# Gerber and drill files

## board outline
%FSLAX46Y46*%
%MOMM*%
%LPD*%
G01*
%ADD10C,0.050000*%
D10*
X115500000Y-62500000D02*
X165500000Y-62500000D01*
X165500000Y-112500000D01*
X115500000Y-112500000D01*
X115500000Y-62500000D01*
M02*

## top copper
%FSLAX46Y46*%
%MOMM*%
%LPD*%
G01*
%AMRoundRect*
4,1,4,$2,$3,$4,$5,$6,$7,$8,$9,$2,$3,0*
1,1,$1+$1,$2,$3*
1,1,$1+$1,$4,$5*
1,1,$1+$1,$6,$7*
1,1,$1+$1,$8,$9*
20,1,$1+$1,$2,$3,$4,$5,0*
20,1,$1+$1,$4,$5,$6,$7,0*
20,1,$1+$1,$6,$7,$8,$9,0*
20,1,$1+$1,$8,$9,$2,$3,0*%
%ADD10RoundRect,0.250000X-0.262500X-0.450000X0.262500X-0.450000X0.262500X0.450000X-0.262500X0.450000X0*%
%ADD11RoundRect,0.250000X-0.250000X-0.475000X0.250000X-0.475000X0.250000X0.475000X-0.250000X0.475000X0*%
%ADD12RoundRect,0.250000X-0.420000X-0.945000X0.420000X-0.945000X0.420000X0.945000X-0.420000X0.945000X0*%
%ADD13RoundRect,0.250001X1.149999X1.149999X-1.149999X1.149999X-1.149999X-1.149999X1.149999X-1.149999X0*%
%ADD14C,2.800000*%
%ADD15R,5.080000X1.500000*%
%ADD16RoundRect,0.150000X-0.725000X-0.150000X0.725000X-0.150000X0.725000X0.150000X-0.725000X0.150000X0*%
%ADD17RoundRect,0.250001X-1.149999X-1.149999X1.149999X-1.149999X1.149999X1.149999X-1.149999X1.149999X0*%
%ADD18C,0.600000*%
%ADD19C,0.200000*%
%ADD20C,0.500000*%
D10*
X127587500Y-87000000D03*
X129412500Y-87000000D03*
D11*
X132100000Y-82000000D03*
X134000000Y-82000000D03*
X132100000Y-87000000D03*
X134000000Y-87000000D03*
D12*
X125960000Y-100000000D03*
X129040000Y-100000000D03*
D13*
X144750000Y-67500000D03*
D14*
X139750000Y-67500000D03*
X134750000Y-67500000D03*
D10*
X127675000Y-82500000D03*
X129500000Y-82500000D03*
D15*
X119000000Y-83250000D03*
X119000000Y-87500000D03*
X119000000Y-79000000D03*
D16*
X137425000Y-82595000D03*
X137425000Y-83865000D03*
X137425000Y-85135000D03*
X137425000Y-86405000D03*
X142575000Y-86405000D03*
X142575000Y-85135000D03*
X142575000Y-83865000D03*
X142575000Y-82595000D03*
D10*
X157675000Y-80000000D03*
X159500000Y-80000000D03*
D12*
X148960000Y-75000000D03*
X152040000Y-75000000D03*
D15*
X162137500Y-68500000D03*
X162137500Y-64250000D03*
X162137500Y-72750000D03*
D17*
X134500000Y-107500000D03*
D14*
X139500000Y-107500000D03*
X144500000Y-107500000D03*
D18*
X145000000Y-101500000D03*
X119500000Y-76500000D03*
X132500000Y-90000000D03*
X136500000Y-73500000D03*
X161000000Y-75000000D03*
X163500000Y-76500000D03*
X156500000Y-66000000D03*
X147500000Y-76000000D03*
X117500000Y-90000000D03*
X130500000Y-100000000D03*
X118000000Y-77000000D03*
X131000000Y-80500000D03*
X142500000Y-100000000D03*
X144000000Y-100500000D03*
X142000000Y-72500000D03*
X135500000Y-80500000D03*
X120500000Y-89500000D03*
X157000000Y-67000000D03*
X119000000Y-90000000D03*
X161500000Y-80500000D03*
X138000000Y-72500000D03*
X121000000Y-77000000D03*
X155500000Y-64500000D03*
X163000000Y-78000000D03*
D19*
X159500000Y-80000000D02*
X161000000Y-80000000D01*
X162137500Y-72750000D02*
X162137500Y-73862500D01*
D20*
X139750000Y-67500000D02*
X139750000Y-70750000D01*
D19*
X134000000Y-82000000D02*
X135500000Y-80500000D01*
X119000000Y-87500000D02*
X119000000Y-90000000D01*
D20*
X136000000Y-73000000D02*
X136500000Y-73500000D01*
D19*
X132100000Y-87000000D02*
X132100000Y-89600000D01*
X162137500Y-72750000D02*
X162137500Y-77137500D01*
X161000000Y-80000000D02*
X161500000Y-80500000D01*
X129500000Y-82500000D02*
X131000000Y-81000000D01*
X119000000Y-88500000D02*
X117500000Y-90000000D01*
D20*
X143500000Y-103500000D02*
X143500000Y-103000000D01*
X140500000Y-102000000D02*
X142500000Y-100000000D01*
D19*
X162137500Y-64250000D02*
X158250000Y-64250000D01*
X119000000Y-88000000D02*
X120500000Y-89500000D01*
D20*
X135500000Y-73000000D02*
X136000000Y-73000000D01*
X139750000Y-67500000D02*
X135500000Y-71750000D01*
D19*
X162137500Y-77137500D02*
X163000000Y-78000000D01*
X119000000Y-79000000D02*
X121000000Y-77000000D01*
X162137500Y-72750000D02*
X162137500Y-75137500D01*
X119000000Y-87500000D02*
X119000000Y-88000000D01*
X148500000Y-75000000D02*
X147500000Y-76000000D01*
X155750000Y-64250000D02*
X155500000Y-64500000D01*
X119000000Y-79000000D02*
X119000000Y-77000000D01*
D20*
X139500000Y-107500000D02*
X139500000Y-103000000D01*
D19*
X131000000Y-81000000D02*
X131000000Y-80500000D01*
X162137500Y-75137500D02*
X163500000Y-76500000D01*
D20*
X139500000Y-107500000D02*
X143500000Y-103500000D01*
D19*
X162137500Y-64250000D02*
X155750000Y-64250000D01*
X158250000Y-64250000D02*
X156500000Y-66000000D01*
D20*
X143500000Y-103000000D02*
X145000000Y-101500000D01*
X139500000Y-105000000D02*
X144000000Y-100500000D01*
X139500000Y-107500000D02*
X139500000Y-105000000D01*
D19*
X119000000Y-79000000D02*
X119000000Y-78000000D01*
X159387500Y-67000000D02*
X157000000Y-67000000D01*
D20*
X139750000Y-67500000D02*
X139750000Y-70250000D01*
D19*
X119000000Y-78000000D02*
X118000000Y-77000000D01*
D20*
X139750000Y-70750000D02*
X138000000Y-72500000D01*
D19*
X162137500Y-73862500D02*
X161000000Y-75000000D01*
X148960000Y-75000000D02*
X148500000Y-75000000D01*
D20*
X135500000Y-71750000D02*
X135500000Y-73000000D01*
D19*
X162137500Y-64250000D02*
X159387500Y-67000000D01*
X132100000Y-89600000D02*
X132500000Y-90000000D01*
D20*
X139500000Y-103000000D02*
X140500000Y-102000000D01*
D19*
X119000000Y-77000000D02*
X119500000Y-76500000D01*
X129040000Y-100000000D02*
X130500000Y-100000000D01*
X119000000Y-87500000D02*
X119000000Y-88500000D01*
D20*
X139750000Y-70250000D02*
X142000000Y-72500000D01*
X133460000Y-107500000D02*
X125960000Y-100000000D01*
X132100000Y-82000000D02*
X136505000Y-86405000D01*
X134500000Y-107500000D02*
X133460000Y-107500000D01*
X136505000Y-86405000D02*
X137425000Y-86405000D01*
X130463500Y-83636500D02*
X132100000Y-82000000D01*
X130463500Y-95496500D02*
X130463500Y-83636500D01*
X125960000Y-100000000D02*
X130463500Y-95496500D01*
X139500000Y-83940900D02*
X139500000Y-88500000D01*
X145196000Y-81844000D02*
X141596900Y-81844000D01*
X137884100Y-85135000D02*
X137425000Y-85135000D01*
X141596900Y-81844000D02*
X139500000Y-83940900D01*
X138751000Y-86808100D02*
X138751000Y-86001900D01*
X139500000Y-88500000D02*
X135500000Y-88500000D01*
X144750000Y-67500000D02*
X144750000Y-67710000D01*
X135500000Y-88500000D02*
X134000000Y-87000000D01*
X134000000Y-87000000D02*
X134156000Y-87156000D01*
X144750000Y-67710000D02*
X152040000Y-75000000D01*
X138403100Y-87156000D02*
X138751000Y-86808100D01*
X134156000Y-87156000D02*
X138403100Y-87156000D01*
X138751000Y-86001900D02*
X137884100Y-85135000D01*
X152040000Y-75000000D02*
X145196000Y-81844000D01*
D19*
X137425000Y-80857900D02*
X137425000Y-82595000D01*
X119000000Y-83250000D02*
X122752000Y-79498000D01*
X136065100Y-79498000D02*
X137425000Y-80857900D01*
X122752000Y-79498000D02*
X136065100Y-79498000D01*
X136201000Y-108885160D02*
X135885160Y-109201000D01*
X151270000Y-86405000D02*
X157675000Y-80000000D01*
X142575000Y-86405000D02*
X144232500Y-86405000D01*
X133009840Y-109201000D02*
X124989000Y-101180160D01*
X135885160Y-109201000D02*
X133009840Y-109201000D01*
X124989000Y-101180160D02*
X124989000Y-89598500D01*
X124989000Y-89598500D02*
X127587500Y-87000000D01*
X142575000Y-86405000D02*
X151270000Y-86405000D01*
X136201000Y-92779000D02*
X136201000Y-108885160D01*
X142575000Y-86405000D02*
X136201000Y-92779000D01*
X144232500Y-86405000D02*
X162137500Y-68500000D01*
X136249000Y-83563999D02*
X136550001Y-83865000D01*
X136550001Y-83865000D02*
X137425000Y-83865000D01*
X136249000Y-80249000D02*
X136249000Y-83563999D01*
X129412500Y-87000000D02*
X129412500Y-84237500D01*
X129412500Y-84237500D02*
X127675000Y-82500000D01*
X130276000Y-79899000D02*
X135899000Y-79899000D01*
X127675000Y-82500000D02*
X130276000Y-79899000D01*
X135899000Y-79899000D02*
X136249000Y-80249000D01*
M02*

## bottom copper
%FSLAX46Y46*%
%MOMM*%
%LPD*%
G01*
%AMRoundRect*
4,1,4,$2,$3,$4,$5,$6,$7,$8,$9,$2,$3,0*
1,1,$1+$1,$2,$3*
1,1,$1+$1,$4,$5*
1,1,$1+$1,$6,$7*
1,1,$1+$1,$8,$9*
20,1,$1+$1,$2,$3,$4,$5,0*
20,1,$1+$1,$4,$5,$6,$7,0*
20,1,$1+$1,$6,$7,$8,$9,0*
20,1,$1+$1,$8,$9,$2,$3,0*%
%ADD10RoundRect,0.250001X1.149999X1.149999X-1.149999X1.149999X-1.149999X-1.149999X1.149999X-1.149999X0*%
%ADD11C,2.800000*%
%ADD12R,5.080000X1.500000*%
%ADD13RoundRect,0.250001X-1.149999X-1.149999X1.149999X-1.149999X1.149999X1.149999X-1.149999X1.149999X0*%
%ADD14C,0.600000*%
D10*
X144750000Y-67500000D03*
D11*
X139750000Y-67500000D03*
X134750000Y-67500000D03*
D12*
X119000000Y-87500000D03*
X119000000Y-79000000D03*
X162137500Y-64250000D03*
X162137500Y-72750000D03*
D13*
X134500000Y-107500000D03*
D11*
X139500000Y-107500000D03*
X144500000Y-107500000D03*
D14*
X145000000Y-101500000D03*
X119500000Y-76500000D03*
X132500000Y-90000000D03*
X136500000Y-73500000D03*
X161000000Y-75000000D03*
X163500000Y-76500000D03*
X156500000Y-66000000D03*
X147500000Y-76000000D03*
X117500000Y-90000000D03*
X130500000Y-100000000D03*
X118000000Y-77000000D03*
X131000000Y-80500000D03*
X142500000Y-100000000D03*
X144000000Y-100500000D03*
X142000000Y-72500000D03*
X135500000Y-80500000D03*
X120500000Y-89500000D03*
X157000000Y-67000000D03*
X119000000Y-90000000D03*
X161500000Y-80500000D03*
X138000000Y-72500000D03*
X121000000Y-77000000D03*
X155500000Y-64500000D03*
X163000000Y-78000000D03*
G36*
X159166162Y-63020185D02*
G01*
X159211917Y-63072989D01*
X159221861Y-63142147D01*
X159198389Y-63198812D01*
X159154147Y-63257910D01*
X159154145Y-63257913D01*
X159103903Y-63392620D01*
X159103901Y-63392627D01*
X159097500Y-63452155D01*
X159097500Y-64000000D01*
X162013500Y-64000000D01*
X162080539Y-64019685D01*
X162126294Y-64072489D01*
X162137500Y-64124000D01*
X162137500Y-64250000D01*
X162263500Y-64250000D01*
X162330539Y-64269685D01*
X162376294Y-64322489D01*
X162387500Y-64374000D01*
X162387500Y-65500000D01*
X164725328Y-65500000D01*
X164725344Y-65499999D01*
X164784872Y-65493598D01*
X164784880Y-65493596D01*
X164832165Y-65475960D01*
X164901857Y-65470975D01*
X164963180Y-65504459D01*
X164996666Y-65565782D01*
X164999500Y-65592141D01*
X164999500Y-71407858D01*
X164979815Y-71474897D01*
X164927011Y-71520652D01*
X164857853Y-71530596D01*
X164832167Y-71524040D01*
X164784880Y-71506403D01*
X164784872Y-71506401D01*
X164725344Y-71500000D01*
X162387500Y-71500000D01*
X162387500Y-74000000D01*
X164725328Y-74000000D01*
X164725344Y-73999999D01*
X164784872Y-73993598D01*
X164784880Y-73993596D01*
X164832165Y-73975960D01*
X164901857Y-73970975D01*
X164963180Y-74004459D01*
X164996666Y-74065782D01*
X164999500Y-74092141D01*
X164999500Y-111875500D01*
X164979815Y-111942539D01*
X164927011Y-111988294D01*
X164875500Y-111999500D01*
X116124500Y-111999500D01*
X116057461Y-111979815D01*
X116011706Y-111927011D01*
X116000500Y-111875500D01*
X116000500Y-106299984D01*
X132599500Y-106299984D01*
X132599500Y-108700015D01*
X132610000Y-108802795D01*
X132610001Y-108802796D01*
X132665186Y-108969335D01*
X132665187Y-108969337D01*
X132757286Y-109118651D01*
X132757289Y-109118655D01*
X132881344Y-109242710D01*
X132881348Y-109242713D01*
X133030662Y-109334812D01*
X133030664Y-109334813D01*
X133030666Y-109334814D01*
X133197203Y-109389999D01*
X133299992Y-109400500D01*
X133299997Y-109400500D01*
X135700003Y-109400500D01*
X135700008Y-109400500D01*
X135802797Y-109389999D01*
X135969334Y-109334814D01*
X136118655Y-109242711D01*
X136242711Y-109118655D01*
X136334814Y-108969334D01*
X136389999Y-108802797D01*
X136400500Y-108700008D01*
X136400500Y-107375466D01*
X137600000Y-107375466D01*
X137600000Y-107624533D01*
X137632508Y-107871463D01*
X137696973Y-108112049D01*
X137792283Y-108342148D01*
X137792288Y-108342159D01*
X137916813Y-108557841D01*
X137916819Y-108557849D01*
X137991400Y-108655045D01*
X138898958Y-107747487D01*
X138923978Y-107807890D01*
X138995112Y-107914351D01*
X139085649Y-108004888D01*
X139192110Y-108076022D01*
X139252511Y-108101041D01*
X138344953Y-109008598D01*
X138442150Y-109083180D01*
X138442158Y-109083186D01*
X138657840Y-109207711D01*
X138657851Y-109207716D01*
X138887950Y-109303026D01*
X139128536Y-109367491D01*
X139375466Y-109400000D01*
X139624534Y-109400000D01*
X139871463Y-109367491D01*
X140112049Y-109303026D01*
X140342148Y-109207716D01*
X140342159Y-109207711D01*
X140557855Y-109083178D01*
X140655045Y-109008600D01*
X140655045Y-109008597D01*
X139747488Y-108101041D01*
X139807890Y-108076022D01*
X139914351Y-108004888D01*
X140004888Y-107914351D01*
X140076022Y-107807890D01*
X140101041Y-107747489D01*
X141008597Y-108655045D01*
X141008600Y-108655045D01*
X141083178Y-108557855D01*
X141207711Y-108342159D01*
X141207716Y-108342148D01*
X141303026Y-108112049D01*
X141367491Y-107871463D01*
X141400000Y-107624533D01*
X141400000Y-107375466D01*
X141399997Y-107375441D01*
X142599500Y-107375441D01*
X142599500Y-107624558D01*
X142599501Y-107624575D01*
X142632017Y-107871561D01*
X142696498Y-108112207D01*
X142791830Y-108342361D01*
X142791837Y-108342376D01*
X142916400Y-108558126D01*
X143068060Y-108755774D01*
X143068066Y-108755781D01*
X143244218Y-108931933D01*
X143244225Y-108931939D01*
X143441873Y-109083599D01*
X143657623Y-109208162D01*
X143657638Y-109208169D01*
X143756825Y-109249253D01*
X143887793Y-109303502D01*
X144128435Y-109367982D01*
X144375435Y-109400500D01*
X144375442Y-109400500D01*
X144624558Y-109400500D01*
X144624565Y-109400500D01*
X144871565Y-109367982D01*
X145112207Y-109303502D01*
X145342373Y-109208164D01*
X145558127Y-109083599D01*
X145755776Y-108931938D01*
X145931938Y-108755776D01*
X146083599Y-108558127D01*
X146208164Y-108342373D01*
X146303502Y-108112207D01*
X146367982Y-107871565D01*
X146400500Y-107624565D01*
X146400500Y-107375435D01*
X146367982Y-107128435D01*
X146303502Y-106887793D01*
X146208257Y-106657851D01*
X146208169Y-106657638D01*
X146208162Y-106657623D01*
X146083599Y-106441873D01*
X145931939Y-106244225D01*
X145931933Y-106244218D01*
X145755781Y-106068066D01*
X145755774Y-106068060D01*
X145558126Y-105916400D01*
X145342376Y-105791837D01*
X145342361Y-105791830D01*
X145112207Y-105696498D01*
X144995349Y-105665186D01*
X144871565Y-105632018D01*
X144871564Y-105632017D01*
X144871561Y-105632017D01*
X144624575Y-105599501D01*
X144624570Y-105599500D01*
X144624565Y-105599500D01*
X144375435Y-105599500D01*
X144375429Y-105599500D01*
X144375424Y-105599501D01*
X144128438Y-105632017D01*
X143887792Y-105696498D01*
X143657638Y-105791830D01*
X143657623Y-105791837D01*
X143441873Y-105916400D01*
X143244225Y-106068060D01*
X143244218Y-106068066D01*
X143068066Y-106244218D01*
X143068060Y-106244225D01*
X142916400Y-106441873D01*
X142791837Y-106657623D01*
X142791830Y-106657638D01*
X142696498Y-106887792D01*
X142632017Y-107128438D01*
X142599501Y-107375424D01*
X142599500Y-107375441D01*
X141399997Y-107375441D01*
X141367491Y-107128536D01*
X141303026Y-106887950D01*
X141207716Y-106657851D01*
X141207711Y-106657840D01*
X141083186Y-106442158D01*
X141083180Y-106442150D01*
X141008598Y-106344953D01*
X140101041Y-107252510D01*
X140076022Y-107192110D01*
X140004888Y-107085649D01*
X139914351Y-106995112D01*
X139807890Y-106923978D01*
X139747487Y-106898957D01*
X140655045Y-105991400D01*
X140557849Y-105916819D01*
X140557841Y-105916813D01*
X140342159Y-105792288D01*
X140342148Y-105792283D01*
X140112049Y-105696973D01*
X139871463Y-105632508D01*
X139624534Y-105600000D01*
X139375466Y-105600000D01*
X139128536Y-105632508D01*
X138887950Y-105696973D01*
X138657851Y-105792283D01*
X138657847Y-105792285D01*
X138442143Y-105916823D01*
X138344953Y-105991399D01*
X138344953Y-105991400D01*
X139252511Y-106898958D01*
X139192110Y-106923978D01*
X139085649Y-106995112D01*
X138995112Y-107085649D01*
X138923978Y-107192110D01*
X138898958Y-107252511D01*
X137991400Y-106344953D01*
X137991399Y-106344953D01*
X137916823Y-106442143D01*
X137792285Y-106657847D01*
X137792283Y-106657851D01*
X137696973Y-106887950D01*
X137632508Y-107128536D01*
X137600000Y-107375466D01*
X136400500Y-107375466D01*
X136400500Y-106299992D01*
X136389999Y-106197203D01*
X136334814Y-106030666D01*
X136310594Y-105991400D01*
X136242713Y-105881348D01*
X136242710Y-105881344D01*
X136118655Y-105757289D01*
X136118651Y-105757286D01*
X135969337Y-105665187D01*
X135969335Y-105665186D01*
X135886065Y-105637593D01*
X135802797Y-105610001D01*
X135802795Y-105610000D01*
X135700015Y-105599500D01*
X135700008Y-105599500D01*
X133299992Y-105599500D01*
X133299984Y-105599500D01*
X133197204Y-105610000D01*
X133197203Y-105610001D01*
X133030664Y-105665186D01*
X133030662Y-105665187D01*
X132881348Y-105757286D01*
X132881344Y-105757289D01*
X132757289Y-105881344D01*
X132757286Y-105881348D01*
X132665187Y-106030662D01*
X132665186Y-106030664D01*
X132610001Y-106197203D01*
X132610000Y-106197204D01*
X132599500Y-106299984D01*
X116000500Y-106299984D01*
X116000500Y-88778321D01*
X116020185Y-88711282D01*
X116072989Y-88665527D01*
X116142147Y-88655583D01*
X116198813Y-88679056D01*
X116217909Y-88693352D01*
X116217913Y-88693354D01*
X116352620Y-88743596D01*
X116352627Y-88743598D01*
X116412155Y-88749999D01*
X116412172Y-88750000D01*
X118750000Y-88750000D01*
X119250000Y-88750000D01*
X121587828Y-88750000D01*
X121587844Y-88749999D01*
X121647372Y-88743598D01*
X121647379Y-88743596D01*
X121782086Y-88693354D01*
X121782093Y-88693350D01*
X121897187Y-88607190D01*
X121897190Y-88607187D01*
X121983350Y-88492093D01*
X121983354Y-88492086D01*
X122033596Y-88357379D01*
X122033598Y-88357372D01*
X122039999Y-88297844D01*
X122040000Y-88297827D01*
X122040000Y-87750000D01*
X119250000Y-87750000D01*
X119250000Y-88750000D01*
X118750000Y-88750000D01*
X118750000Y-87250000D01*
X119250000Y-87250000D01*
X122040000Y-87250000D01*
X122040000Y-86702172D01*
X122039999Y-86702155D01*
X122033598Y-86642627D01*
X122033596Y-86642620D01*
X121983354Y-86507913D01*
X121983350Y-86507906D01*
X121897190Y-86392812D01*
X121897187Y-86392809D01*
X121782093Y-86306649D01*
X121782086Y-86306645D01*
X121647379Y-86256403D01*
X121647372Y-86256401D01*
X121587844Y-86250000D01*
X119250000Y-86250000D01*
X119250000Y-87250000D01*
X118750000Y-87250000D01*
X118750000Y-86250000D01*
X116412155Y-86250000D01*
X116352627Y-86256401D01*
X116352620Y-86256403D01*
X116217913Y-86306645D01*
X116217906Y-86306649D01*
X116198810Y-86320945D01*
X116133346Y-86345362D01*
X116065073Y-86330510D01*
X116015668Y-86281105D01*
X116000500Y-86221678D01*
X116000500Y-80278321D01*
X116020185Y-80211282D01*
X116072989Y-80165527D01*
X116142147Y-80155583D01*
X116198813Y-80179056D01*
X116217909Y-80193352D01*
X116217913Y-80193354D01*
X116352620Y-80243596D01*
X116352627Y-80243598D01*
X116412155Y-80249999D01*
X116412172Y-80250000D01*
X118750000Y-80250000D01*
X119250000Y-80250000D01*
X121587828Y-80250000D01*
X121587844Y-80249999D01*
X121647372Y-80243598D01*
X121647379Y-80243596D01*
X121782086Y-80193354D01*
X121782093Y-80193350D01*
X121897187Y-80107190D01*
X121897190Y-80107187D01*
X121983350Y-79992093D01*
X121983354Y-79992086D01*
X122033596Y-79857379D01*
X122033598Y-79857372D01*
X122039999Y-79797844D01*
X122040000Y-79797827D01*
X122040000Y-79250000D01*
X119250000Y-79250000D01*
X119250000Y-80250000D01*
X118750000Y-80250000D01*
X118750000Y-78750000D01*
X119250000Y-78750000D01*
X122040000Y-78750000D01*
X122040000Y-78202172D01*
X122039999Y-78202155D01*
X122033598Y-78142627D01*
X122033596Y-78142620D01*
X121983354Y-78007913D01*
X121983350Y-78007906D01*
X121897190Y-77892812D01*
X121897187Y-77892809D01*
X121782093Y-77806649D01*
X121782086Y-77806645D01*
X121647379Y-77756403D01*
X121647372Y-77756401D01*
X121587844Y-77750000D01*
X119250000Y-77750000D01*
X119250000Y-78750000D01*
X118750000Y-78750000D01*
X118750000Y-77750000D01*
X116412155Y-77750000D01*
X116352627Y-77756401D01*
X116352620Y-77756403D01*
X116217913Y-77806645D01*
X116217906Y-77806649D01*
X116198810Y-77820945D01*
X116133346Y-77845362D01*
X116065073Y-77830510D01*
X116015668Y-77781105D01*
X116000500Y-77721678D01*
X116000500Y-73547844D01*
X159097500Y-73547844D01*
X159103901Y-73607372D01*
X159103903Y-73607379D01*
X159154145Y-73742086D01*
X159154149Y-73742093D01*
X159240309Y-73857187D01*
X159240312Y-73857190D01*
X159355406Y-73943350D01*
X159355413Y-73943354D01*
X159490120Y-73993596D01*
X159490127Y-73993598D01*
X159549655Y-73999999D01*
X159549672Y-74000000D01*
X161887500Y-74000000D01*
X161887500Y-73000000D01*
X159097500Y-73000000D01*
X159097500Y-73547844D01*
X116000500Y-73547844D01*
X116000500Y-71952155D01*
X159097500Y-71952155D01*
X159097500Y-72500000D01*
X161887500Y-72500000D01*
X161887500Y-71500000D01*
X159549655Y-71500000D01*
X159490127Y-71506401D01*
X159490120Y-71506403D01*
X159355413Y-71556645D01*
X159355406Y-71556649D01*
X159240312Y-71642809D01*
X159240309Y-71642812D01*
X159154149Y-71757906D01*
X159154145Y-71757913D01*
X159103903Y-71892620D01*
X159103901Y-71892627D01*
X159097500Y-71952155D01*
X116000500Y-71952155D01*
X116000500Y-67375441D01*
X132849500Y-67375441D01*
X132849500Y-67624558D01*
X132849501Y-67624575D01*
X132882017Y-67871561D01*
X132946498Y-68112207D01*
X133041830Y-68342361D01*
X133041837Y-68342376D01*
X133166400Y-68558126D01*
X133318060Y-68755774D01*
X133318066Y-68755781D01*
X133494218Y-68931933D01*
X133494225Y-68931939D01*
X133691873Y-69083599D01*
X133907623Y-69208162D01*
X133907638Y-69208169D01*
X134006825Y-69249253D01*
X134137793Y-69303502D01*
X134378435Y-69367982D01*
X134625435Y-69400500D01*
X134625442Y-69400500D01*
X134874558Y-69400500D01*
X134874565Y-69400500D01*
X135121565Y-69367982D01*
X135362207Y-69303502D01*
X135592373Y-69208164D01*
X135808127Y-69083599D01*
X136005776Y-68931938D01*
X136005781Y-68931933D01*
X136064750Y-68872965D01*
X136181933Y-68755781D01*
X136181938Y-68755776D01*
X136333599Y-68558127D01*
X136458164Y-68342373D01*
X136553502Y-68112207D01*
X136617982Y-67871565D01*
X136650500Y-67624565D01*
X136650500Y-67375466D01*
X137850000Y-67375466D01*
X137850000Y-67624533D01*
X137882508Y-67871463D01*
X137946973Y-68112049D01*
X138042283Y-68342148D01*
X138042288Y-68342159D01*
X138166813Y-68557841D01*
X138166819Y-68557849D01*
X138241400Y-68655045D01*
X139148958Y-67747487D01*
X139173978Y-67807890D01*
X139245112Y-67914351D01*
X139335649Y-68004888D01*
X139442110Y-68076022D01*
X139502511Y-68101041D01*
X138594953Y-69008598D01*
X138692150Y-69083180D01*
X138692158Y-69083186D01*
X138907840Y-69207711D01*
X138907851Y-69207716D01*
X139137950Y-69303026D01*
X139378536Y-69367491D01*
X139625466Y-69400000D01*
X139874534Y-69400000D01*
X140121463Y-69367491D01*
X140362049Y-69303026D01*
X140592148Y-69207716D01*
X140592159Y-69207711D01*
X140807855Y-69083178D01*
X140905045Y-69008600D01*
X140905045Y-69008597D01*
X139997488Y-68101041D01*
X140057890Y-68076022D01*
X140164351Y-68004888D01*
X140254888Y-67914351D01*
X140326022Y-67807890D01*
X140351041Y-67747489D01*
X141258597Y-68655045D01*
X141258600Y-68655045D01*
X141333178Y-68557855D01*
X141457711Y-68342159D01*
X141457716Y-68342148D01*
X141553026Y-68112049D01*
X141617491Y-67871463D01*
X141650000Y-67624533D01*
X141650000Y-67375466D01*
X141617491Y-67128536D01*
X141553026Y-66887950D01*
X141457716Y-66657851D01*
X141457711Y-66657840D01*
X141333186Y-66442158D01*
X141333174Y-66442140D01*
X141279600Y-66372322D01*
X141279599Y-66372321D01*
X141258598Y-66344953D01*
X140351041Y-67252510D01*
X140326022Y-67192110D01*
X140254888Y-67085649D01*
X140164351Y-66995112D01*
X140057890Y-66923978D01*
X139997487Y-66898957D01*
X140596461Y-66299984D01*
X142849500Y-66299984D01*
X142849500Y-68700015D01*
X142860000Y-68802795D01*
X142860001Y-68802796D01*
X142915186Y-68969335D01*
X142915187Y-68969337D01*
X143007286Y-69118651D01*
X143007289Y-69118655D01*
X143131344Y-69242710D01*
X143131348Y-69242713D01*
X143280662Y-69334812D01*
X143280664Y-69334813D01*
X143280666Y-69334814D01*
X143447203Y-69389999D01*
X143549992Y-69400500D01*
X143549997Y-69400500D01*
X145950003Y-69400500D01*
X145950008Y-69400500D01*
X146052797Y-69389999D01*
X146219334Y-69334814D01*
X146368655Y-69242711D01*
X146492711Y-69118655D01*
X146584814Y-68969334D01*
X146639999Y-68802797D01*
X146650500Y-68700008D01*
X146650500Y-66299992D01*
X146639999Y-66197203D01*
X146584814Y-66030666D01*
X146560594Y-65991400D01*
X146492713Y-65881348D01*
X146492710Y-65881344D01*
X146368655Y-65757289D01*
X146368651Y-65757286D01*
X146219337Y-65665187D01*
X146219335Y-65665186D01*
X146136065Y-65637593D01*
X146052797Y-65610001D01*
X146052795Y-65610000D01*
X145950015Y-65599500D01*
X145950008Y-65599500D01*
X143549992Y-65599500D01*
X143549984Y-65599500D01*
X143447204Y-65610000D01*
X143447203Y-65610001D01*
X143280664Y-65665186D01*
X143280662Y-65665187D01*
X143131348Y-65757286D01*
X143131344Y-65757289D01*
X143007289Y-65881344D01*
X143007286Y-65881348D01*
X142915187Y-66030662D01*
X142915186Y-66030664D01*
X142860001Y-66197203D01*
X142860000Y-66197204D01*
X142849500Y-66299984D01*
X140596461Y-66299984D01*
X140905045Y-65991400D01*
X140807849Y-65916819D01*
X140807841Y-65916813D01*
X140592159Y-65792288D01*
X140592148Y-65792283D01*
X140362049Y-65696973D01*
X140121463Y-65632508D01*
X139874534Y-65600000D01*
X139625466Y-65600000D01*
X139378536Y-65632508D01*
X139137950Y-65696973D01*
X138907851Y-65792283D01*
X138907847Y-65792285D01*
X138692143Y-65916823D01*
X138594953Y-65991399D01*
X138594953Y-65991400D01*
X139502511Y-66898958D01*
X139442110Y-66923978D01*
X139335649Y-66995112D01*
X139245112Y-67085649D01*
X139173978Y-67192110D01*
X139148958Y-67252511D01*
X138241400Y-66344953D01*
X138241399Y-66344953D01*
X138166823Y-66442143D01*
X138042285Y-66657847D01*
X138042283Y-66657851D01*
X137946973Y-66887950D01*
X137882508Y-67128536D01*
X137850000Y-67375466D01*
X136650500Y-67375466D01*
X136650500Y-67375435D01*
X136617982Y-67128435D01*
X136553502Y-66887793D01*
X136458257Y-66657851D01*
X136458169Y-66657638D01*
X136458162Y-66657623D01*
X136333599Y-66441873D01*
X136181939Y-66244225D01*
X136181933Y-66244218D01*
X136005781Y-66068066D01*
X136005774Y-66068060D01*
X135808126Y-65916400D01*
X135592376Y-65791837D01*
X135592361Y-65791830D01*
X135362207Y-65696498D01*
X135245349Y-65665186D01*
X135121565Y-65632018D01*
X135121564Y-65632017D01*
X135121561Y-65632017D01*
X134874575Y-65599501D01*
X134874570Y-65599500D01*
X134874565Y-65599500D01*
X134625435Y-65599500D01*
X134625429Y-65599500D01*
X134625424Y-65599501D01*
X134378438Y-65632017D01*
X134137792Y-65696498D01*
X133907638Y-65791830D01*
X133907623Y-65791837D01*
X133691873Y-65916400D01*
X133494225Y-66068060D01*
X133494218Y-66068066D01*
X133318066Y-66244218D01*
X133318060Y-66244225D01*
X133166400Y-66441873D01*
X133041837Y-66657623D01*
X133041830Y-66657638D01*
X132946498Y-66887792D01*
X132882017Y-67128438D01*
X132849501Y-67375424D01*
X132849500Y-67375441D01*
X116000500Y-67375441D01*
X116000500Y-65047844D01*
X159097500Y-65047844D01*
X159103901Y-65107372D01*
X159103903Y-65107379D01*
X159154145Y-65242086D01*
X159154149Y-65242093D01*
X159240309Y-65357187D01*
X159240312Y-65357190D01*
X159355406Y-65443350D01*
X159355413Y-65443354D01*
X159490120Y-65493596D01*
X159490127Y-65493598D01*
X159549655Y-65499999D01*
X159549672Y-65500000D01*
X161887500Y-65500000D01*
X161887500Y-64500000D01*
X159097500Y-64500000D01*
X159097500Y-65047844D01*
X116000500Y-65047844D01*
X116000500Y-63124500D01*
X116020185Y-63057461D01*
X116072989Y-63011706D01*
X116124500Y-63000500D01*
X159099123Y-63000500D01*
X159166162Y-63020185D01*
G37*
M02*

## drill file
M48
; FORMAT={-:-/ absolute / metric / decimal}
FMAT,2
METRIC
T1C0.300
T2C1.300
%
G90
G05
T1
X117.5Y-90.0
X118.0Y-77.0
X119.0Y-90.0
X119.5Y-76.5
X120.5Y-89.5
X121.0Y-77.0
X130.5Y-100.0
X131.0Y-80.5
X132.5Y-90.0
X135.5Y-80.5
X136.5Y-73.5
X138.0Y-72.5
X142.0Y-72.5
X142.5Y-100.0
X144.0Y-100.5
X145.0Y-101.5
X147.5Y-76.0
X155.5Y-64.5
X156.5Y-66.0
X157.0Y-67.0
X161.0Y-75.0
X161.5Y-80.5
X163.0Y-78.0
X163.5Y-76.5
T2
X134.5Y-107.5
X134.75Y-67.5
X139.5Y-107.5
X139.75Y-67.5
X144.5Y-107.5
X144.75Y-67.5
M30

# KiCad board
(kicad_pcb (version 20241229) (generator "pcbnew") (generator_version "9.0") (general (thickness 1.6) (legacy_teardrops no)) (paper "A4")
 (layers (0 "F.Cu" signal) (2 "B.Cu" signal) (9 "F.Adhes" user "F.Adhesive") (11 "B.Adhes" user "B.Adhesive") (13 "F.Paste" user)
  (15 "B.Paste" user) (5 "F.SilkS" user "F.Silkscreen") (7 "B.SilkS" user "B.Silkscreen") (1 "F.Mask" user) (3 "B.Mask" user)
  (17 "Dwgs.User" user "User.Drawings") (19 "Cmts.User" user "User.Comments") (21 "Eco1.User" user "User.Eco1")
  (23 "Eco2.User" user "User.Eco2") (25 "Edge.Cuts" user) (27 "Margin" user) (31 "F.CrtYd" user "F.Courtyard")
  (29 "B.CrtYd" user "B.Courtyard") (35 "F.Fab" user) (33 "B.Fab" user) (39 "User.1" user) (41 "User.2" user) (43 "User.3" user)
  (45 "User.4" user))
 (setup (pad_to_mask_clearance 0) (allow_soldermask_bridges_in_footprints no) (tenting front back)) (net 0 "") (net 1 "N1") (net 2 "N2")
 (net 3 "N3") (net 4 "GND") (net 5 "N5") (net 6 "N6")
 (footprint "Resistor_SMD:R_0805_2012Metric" (layer "F.Cu") (at 128.5 87)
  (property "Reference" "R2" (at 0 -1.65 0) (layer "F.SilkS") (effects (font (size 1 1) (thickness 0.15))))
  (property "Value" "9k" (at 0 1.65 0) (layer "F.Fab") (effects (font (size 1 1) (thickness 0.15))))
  (pad "1" smd roundrect (at -0.9125 0) (size 1.025 1.4) (layers "F.Cu" "F.Mask" "F.Paste") (roundrect_rratio 0.243902) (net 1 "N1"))
  (pad "2" smd roundrect (at 0.9125 0) (size 1.025 1.4) (layers "F.Cu" "F.Mask" "F.Paste") (roundrect_rratio 0.243902) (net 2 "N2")))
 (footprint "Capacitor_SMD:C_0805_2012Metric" (layer "F.Cu") (at 133.05 82)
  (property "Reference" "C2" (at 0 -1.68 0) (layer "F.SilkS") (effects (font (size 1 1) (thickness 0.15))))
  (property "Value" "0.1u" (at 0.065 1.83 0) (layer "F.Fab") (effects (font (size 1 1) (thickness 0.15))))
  (pad "1" smd roundrect (at -0.95 0) (size 1 1.45) (layers "F.Cu" "F.Mask" "F.Paste") (roundrect_rratio 0.25) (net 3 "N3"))
  (pad "2" smd roundrect (at 0.95 0) (size 1 1.45) (layers "F.Cu" "F.Mask" "F.Paste") (roundrect_rratio 0.25) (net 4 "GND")))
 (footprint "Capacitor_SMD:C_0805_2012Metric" (layer "F.Cu") (at 133.05 87)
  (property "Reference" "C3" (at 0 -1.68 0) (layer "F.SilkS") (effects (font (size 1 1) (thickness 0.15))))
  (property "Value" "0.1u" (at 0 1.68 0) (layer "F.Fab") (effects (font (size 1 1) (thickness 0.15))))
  (pad "1" smd roundrect (at -0.95 0) (size 1 1.45) (layers "F.Cu" "F.Mask" "F.Paste") (roundrect_rratio 0.25) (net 4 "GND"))
  (pad "2" smd roundrect (at 0.95 0) (size 1 1.45) (layers "F.Cu" "F.Mask" "F.Paste") (roundrect_rratio 0.25) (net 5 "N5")))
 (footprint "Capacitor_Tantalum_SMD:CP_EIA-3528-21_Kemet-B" (layer "F.Cu") (at 127.5 100)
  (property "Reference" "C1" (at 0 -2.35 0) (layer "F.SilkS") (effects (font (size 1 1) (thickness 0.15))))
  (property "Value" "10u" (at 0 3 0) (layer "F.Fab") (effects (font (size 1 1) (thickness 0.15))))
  (pad "1" smd roundrect (at -1.54 0) (size 1.34 2.39) (layers "F.Cu" "F.Mask" "F.Paste") (roundrect_rratio 0.186567) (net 3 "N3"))
  (pad "2" smd roundrect (at 1.54 0) (size 1.34 2.39) (layers "F.Cu" "F.Mask" "F.Paste") (roundrect_rratio 0.186567) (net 4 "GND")))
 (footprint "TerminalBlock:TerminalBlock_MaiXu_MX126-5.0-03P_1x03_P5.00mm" (layer "F.Cu") (at 144.75 67.5 180)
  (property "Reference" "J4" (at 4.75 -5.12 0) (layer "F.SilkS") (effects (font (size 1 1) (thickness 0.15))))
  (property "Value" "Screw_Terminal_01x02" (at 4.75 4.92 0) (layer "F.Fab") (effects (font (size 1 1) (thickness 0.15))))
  (pad "1" thru_hole roundrect (at 0 0 180) (size 2.8 2.8) (drill 1.3) (layers "*.Cu" "*.Mask") (remove_unused_layers no)
   (roundrect_rratio 0.089286) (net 5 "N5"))
  (pad "2" thru_hole circle (at 5 0 180) (size 2.8 2.8) (drill 1.3) (layers "*.Cu" "*.Mask") (remove_unused_layers no) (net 4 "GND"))
  (pad "3" thru_hole circle (at 10 0 180) (size 2.8 2.8) (drill 1.3) (layers "*.Cu" "*.Mask") (remove_unused_layers no)))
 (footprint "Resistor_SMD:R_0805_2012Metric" (layer "F.Cu") (at 128.5875 82.5)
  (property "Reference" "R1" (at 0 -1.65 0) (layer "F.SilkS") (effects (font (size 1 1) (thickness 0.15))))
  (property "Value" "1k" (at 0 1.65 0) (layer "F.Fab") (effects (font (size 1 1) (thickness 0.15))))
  (pad "1" smd roundrect (at -0.9125 0) (size 1.025 1.4) (layers "F.Cu" "F.Mask" "F.Paste") (roundrect_rratio 0.243902) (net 2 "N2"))
  (pad "2" smd roundrect (at 0.9125 0) (size 1.025 1.4) (layers "F.Cu" "F.Mask" "F.Paste") (roundrect_rratio 0.243902) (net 4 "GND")))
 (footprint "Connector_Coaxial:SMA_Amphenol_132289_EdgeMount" (layer "F.Cu") (at 119 83.25 180)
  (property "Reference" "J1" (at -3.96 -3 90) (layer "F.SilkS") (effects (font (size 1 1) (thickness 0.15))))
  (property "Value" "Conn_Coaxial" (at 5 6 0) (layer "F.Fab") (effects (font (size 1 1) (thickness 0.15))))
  (pad "1" smd rect (at 0 0 270) (size 1.5 5.08) (layers "F.Cu" "F.Mask" "F.Paste") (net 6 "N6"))
  (pad "2" smd rect (at 0 -4.25 270) (size 1.5 5.08) (layers "F.Cu" "F.Mask" "F.Paste") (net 4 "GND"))
  (pad "2" smd rect (at 0 -4.25 270) (size 1.5 5.08) (layers "B.Cu" "B.Mask" "B.Paste") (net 4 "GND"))
  (pad "2" smd rect (at 0 4.25 270) (size 1.5 5.08) (layers "F.Cu" "F.Mask" "F.Paste") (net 4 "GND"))
  (pad "2" smd rect (at 0 4.25 270) (size 1.5 5.08) (layers "B.Cu" "B.Mask" "B.Paste") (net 4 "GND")))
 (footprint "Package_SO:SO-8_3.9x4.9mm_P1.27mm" (layer "F.Cu") (at 140 84.5)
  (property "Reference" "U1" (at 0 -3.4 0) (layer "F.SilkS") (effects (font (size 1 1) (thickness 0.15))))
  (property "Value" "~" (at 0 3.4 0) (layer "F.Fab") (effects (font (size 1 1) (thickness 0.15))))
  (pad "1" smd roundrect (at -2.575 -1.905) (size 1.75 0.6) (layers "F.Cu" "F.Mask" "F.Paste") (roundrect_rratio 0.25) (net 6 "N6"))
  (pad "2" smd roundrect (at -2.575 -0.635) (size 1.75 0.6) (layers "F.Cu" "F.Mask" "F.Paste") (roundrect_rratio 0.25) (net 2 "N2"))
  (pad "3" smd roundrect (at -2.575 0.635) (size 1.75 0.6) (layers "F.Cu" "F.Mask" "F.Paste") (roundrect_rratio 0.25) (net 5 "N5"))
  (pad "4" smd roundrect (at -2.575 1.905) (size 1.75 0.6) (layers "F.Cu" "F.Mask" "F.Paste") (roundrect_rratio 0.25) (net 3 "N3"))
  (pad "5" smd roundrect (at 2.575 1.905) (size 1.75 0.6) (layers "F.Cu" "F.Mask" "F.Paste") (roundrect_rratio 0.25) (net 1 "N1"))
  (pad "6" smd roundrect (at 2.575 0.635) (size 1.75 0.6) (layers "F.Cu" "F.Mask" "F.Paste") (roundrect_rratio 0.25))
  (pad "7" smd roundrect (at 2.575 -0.635) (size 1.75 0.6) (layers "F.Cu" "F.Mask" "F.Paste") (roundrect_rratio 0.25))
  (pad "8" smd roundrect (at 2.575 -1.905) (size 1.75 0.6) (layers "F.Cu" "F.Mask" "F.Paste") (roundrect_rratio 0.25)))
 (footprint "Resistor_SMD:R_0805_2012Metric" (layer "F.Cu") (at 158.5875 80)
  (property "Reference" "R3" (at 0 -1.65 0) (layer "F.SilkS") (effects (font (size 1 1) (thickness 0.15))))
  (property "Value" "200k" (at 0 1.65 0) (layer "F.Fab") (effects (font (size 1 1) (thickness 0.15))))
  (pad "1" smd roundrect (at -0.9125 0) (size 1.025 1.4) (layers "F.Cu" "F.Mask" "F.Paste") (roundrect_rratio 0.243902) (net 1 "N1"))
  (pad "2" smd roundrect (at 0.9125 0) (size 1.025 1.4) (layers "F.Cu" "F.Mask" "F.Paste") (roundrect_rratio 0.243902) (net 4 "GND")))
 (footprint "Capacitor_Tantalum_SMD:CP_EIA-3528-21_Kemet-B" (layer "F.Cu") (at 150.5 75)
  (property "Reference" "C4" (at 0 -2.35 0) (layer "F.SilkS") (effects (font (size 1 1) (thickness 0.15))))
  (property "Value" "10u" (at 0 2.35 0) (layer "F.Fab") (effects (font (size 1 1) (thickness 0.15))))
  (pad "1" smd roundrect (at -1.54 0) (size 1.34 2.39) (layers "F.Cu" "F.Mask" "F.Paste") (roundrect_rratio 0.186567) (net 4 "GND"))
  (pad "2" smd roundrect (at 1.54 0) (size 1.34 2.39) (layers "F.Cu" "F.Mask" "F.Paste") (roundrect_rratio 0.186567) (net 5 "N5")))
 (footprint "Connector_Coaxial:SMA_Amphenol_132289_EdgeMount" (layer "F.Cu") (at 162.1375 68.5)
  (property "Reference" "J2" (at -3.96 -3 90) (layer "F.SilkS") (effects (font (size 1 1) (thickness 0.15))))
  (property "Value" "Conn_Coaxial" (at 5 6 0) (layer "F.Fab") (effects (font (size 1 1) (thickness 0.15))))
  (pad "1" smd rect (at 0 0 90) (size 1.5 5.08) (layers "F.Cu" "F.Mask" "F.Paste") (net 1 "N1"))
  (pad "2" smd rect (at 0 -4.25 90) (size 1.5 5.08) (layers "F.Cu" "F.Mask" "F.Paste") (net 4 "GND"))
  (pad "2" smd rect (at 0 -4.25 90) (size 1.5 5.08) (layers "B.Cu" "B.Mask" "B.Paste") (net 4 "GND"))
  (pad "2" smd rect (at 0 4.25 90) (size 1.5 5.08) (layers "F.Cu" "F.Mask" "F.Paste") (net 4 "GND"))
  (pad "2" smd rect (at 0 4.25 90) (size 1.5 5.08) (layers "B.Cu" "B.Mask" "B.Paste") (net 4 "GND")))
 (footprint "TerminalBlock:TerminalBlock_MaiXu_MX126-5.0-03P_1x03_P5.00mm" (layer "F.Cu") (at 134.5 107.5)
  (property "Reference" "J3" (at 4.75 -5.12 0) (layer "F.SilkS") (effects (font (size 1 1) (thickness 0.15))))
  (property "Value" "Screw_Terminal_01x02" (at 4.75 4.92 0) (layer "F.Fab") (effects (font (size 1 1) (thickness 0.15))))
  (pad "1" thru_hole roundrect (at 0 0) (size 2.8 2.8) (drill 1.3) (layers "*.Cu" "*.Mask") (remove_unused_layers no)
   (roundrect_rratio 0.089286) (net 3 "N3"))
  (pad "2" thru_hole circle (at 5 0) (size 2.8 2.8) (drill 1.3) (layers "*.Cu" "*.Mask") (remove_unused_layers no) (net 4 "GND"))
  (pad "3" thru_hole circle (at 10 0) (size 2.8 2.8) (drill 1.3) (layers "*.Cu" "*.Mask") (remove_unused_layers no)))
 (gr_rect (start 115.5 62.5) (end 165.5 112.5) (stroke (width 0.05) (type default)) (fill no) (layer "Edge.Cuts"))
 (segment (start 159.5 80) (end 161 80) (width 0.2) (layer "F.Cu") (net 4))
 (segment (start 162.1375 72.75) (end 162.1375 73.8625) (width 0.2) (layer "F.Cu") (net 4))
 (segment (start 139.75 67.5) (end 139.75 70.75) (width 0.5) (layer "F.Cu") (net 4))
 (segment (start 134 82) (end 135.5 80.5) (width 0.2) (layer "F.Cu") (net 4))
 (segment (start 119 87.5) (end 119 90) (width 0.2) (layer "F.Cu") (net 4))
 (segment (start 136 73) (end 136.5 73.5) (width 0.5) (layer "F.Cu") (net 4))
 (segment (start 132.1 87) (end 132.1 89.6) (width 0.2) (layer "F.Cu") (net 4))
 (segment (start 162.1375 72.75) (end 162.1375 77.1375) (width 0.2) (layer "F.Cu") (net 4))
 (segment (start 161 80) (end 161.5 80.5) (width 0.2) (layer "F.Cu") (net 4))
 (segment (start 129.5 82.5) (end 131 81) (width 0.2) (layer "F.Cu") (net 4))
 (segment (start 119 88.5) (end 117.5 90) (width 0.2) (layer "F.Cu") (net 4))
 (segment (start 143.5 103.5) (end 143.5 103) (width 0.5) (layer "F.Cu") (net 4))
 (segment (start 140.5 102) (end 142.5 100) (width 0.5) (layer "F.Cu") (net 4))
 (segment (start 162.1375 64.25) (end 158.25 64.25) (width 0.2) (layer "F.Cu") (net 4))
 (segment (start 119 88) (end 120.5 89.5) (width 0.2) (layer "F.Cu") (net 4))
 (segment (start 135.5 73) (end 136 73) (width 0.5) (layer "F.Cu") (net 4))
 (segment (start 139.75 67.5) (end 135.5 71.75) (width 0.5) (layer "F.Cu") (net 4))
 (segment (start 162.1375 77.1375) (end 163 78) (width 0.2) (layer "F.Cu") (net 4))
 (segment (start 119 79) (end 121 77) (width 0.2) (layer "F.Cu") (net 4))
 (segment (start 162.1375 72.75) (end 162.1375 75.1375) (width 0.2) (layer "F.Cu") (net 4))
 (segment (start 119 87.5) (end 119 88) (width 0.2) (layer "F.Cu") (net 4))
 (segment (start 148.5 75) (end 147.5 76) (width 0.2) (layer "F.Cu") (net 4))
 (segment (start 155.75 64.25) (end 155.5 64.5) (width 0.2) (layer "F.Cu") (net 4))
 (segment (start 119 79) (end 119 77) (width 0.2) (layer "F.Cu") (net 4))
 (segment (start 139.5 107.5) (end 139.5 103) (width 0.5) (layer "F.Cu") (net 4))
 (segment (start 131 81) (end 131 80.5) (width 0.2) (layer "F.Cu") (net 4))
 (segment (start 162.1375 75.1375) (end 163.5 76.5) (width 0.2) (layer "F.Cu") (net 4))
 (segment (start 139.5 107.5) (end 143.5 103.5) (width 0.5) (layer "F.Cu") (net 4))
 (segment (start 162.1375 64.25) (end 155.75 64.25) (width 0.2) (layer "F.Cu") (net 4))
 (segment (start 158.25 64.25) (end 156.5 66) (width 0.2) (layer "F.Cu") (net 4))
 (segment (start 143.5 103) (end 145 101.5) (width 0.5) (layer "F.Cu") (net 4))
 (segment (start 139.5 105) (end 144 100.5) (width 0.5) (layer "F.Cu") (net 4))
 (segment (start 139.5 107.5) (end 139.5 105) (width 0.5) (layer "F.Cu") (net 4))
 (segment (start 119 79) (end 119 78) (width 0.2) (layer "F.Cu") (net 4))
 (segment (start 159.3875 67) (end 157 67) (width 0.2) (layer "F.Cu") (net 4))
 (segment (start 139.75 67.5) (end 139.75 70.25) (width 0.5) (layer "F.Cu") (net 4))
 (segment (start 119 78) (end 118 77) (width 0.2) (layer "F.Cu") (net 4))
 (segment (start 139.75 70.75) (end 138 72.5) (width 0.5) (layer "F.Cu") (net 4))
 (segment (start 162.1375 73.8625) (end 161 75) (width 0.2) (layer "F.Cu") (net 4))
 (segment (start 148.96 75) (end 148.5 75) (width 0.2) (layer "F.Cu") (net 4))
 (segment (start 135.5 71.75) (end 135.5 73) (width 0.5) (layer "F.Cu") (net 4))
 (segment (start 162.1375 64.25) (end 159.3875 67) (width 0.2) (layer "F.Cu") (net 4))
 (segment (start 132.1 89.6) (end 132.5 90) (width 0.2) (layer "F.Cu") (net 4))
 (segment (start 139.5 103) (end 140.5 102) (width 0.5) (layer "F.Cu") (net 4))
 (segment (start 119 77) (end 119.5 76.5) (width 0.2) (layer "F.Cu") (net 4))
 (segment (start 129.04 100) (end 130.5 100) (width 0.2) (layer "F.Cu") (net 4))
 (segment (start 119 87.5) (end 119 88.5) (width 0.2) (layer "F.Cu") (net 4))
 (segment (start 139.75 70.25) (end 142 72.5) (width 0.5) (layer "F.Cu") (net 4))
 (via (at 145 101.5) (size 0.6) (drill 0.3) (layers "F.Cu" "B.Cu") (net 4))
 (via (at 119.5 76.5) (size 0.6) (drill 0.3) (layers "F.Cu" "B.Cu") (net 4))
 (via (at 132.5 90) (size 0.6) (drill 0.3) (layers "F.Cu" "B.Cu") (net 4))
 (via (at 136.5 73.5) (size 0.6) (drill 0.3) (layers "F.Cu" "B.Cu") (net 4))
 (via (at 161 75) (size 0.6) (drill 0.3) (layers "F.Cu" "B.Cu") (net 4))
 (via (at 163.5 76.5) (size 0.6) (drill 0.3) (layers "F.Cu" "B.Cu") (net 4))
 (via (at 156.5 66) (size 0.6) (drill 0.3) (layers "F.Cu" "B.Cu") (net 4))
 (via (at 147.5 76) (size 0.6) (drill 0.3) (layers "F.Cu" "B.Cu") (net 4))
 (via (at 117.5 90) (size 0.6) (drill 0.3) (layers "F.Cu" "B.Cu") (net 4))
 (via (at 130.5 100) (size 0.6) (drill 0.3) (layers "F.Cu" "B.Cu") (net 4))
 (via (at 118 77) (size 0.6) (drill 0.3) (layers "F.Cu" "B.Cu") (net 4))
 (via (at 131 80.5) (size 0.6) (drill 0.3) (layers "F.Cu" "B.Cu") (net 4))
 (via (at 142.5 100) (size 0.6) (drill 0.3) (layers "F.Cu" "B.Cu") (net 4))
 (via (at 144 100.5) (size 0.6) (drill 0.3) (layers "F.Cu" "B.Cu") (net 4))
 (via (at 142 72.5) (size 0.6) (drill 0.3) (layers "F.Cu" "B.Cu") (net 4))
 (via (at 135.5 80.5) (size 0.6) (drill 0.3) (layers "F.Cu" "B.Cu") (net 4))
 (via (at 120.5 89.5) (size 0.6) (drill 0.3) (layers "F.Cu" "B.Cu") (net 4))
 (via (at 157 67) (size 0.6) (drill 0.3) (layers "F.Cu" "B.Cu") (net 4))
 (via (at 119 90) (size 0.6) (drill 0.3) (layers "F.Cu" "B.Cu") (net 4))
 (via (at 161.5 80.5) (size 0.6) (drill 0.3) (layers "F.Cu" "B.Cu") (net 4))
 (via (at 138 72.5) (size 0.6) (drill 0.3) (layers "F.Cu" "B.Cu") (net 4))
 (via (at 121 77) (size 0.6) (drill 0.3) (layers "F.Cu" "B.Cu") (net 4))
 (via (at 155.5 64.5) (size 0.6) (drill 0.3) (layers "F.Cu" "B.Cu") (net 4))
 (via (at 163 78) (size 0.6) (drill 0.3) (layers "F.Cu" "B.Cu") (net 4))
 (segment (start 133.46 107.5) (end 125.96 100) (width 0.5) (layer "F.Cu") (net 3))
 (segment (start 132.1 82) (end 136.505 86.405) (width 0.5) (layer "F.Cu") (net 3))
 (segment (start 134.5 107.5) (end 133.46 107.5) (width 0.5) (layer "F.Cu") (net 3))
 (segment (start 136.505 86.405) (end 137.425 86.405) (width 0.5) (layer "F.Cu") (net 3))
 (segment (start 130.4635 83.6365) (end 132.1 82) (width 0.5) (layer "F.Cu") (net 3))
 (segment (start 130.4635 95.4965) (end 130.4635 83.6365) (width 0.5) (layer "F.Cu") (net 3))
 (segment (start 125.96 100) (end 130.4635 95.4965) (width 0.5) (layer "F.Cu") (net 3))
 (segment (start 139.5 83.9409) (end 139.5 88.5) (width 0.5) (layer "F.Cu") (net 5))
 (segment (start 145.196 81.844) (end 141.5969 81.844) (width 0.5) (layer "F.Cu") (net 5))
 (segment (start 137.8841 85.135) (end 137.425 85.135) (width 0.5) (layer "F.Cu") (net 5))
 (segment (start 141.5969 81.844) (end 139.5 83.9409) (width 0.5) (layer "F.Cu") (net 5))
 (segment (start 138.751 86.8081) (end 138.751 86.0019) (width 0.5) (layer "F.Cu") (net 5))
 (segment (start 139.5 88.5) (end 135.5 88.5) (width 0.5) (layer "F.Cu") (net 5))
 (segment (start 144.75 67.5) (end 144.75 67.71) (width 0.5) (layer "F.Cu") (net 5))
 (segment (start 135.5 88.5) (end 134 87) (width 0.5) (layer "F.Cu") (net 5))
 (segment (start 134 87) (end 134.156 87.156) (width 0.5) (layer "F.Cu") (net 5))
 (segment (start 144.75 67.71) (end 152.04 75) (width 0.5) (layer "F.Cu") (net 5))
 (segment (start 138.4031 87.156) (end 138.751 86.8081) (width 0.5) (layer "F.Cu") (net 5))
 (segment (start 134.156 87.156) (end 138.4031 87.156) (width 0.5) (layer "F.Cu") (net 5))
 (segment (start 138.751 86.0019) (end 137.8841 85.135) (width 0.5) (layer "F.Cu") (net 5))
 (segment (start 152.04 75) (end 145.196 81.844) (width 0.5) (layer "F.Cu") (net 5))
 (segment (start 137.425 80.8579) (end 137.425 82.595) (width 0.2) (layer "F.Cu") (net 6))
 (segment (start 119 83.25) (end 122.752 79.498) (width 0.2) (layer "F.Cu") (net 6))
 (segment (start 136.0651 79.498) (end 137.425 80.8579) (width 0.2) (layer "F.Cu") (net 6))
 (segment (start 122.752 79.498) (end 136.0651 79.498) (width 0.2) (layer "F.Cu") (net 6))
 (segment (start 136.201 108.88516) (end 135.88516 109.201) (width 0.2) (layer "F.Cu") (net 1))
 (segment (start 151.27 86.405) (end 157.675 80) (width 0.2) (layer "F.Cu") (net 1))
 (segment (start 142.575 86.405) (end 144.2325 86.405) (width 0.2) (layer "F.Cu") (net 1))
 (segment (start 133.00984 109.201) (end 124.989 101.18016) (width 0.2) (layer "F.Cu") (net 1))
 (segment (start 135.88516 109.201) (end 133.00984 109.201) (width 0.2) (layer "F.Cu") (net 1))
 (segment (start 124.989 101.18016) (end 124.989 89.5985) (width 0.2) (layer "F.Cu") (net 1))
 (segment (start 124.989 89.5985) (end 127.5875 87) (width 0.2) (layer "F.Cu") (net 1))
 (segment (start 142.575 86.405) (end 151.27 86.405) (width 0.2) (layer "F.Cu") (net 1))
 (segment (start 136.201 92.779) (end 136.201 108.88516) (width 0.2) (layer "F.Cu") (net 1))
 (segment (start 142.575 86.405) (end 136.201 92.779) (width 0.2) (layer "F.Cu") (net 1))
 (segment (start 144.2325 86.405) (end 162.1375 68.5) (width 0.2) (layer "F.Cu") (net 1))
 (segment (start 136.249 83.563999) (end 136.550001 83.865) (width 0.2) (layer "F.Cu") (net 2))
 (segment (start 136.550001 83.865) (end 137.425 83.865) (width 0.2) (layer "F.Cu") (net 2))
 (segment (start 136.249 80.249) (end 136.249 83.563999) (width 0.2) (layer "F.Cu") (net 2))
 (segment (start 129.4125 87) (end 129.4125 84.2375) (width 0.2) (layer "F.Cu") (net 2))
 (segment (start 129.4125 84.2375) (end 127.675 82.5) (width 0.2) (layer "F.Cu") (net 2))
 (segment (start 130.276 79.899) (end 135.899 79.899) (width 0.2) (layer "F.Cu") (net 2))
 (segment (start 127.675 82.5) (end 130.276 79.899) (width 0.2) (layer "F.Cu") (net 2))
 (segment (start 135.899 79.899) (end 136.249 80.249) (width 0.2) (layer "F.Cu") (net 2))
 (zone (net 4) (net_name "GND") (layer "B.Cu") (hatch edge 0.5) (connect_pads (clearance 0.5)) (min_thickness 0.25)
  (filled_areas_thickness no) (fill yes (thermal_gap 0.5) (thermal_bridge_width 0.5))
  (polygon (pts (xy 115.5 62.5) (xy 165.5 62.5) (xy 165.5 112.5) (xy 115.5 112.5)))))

